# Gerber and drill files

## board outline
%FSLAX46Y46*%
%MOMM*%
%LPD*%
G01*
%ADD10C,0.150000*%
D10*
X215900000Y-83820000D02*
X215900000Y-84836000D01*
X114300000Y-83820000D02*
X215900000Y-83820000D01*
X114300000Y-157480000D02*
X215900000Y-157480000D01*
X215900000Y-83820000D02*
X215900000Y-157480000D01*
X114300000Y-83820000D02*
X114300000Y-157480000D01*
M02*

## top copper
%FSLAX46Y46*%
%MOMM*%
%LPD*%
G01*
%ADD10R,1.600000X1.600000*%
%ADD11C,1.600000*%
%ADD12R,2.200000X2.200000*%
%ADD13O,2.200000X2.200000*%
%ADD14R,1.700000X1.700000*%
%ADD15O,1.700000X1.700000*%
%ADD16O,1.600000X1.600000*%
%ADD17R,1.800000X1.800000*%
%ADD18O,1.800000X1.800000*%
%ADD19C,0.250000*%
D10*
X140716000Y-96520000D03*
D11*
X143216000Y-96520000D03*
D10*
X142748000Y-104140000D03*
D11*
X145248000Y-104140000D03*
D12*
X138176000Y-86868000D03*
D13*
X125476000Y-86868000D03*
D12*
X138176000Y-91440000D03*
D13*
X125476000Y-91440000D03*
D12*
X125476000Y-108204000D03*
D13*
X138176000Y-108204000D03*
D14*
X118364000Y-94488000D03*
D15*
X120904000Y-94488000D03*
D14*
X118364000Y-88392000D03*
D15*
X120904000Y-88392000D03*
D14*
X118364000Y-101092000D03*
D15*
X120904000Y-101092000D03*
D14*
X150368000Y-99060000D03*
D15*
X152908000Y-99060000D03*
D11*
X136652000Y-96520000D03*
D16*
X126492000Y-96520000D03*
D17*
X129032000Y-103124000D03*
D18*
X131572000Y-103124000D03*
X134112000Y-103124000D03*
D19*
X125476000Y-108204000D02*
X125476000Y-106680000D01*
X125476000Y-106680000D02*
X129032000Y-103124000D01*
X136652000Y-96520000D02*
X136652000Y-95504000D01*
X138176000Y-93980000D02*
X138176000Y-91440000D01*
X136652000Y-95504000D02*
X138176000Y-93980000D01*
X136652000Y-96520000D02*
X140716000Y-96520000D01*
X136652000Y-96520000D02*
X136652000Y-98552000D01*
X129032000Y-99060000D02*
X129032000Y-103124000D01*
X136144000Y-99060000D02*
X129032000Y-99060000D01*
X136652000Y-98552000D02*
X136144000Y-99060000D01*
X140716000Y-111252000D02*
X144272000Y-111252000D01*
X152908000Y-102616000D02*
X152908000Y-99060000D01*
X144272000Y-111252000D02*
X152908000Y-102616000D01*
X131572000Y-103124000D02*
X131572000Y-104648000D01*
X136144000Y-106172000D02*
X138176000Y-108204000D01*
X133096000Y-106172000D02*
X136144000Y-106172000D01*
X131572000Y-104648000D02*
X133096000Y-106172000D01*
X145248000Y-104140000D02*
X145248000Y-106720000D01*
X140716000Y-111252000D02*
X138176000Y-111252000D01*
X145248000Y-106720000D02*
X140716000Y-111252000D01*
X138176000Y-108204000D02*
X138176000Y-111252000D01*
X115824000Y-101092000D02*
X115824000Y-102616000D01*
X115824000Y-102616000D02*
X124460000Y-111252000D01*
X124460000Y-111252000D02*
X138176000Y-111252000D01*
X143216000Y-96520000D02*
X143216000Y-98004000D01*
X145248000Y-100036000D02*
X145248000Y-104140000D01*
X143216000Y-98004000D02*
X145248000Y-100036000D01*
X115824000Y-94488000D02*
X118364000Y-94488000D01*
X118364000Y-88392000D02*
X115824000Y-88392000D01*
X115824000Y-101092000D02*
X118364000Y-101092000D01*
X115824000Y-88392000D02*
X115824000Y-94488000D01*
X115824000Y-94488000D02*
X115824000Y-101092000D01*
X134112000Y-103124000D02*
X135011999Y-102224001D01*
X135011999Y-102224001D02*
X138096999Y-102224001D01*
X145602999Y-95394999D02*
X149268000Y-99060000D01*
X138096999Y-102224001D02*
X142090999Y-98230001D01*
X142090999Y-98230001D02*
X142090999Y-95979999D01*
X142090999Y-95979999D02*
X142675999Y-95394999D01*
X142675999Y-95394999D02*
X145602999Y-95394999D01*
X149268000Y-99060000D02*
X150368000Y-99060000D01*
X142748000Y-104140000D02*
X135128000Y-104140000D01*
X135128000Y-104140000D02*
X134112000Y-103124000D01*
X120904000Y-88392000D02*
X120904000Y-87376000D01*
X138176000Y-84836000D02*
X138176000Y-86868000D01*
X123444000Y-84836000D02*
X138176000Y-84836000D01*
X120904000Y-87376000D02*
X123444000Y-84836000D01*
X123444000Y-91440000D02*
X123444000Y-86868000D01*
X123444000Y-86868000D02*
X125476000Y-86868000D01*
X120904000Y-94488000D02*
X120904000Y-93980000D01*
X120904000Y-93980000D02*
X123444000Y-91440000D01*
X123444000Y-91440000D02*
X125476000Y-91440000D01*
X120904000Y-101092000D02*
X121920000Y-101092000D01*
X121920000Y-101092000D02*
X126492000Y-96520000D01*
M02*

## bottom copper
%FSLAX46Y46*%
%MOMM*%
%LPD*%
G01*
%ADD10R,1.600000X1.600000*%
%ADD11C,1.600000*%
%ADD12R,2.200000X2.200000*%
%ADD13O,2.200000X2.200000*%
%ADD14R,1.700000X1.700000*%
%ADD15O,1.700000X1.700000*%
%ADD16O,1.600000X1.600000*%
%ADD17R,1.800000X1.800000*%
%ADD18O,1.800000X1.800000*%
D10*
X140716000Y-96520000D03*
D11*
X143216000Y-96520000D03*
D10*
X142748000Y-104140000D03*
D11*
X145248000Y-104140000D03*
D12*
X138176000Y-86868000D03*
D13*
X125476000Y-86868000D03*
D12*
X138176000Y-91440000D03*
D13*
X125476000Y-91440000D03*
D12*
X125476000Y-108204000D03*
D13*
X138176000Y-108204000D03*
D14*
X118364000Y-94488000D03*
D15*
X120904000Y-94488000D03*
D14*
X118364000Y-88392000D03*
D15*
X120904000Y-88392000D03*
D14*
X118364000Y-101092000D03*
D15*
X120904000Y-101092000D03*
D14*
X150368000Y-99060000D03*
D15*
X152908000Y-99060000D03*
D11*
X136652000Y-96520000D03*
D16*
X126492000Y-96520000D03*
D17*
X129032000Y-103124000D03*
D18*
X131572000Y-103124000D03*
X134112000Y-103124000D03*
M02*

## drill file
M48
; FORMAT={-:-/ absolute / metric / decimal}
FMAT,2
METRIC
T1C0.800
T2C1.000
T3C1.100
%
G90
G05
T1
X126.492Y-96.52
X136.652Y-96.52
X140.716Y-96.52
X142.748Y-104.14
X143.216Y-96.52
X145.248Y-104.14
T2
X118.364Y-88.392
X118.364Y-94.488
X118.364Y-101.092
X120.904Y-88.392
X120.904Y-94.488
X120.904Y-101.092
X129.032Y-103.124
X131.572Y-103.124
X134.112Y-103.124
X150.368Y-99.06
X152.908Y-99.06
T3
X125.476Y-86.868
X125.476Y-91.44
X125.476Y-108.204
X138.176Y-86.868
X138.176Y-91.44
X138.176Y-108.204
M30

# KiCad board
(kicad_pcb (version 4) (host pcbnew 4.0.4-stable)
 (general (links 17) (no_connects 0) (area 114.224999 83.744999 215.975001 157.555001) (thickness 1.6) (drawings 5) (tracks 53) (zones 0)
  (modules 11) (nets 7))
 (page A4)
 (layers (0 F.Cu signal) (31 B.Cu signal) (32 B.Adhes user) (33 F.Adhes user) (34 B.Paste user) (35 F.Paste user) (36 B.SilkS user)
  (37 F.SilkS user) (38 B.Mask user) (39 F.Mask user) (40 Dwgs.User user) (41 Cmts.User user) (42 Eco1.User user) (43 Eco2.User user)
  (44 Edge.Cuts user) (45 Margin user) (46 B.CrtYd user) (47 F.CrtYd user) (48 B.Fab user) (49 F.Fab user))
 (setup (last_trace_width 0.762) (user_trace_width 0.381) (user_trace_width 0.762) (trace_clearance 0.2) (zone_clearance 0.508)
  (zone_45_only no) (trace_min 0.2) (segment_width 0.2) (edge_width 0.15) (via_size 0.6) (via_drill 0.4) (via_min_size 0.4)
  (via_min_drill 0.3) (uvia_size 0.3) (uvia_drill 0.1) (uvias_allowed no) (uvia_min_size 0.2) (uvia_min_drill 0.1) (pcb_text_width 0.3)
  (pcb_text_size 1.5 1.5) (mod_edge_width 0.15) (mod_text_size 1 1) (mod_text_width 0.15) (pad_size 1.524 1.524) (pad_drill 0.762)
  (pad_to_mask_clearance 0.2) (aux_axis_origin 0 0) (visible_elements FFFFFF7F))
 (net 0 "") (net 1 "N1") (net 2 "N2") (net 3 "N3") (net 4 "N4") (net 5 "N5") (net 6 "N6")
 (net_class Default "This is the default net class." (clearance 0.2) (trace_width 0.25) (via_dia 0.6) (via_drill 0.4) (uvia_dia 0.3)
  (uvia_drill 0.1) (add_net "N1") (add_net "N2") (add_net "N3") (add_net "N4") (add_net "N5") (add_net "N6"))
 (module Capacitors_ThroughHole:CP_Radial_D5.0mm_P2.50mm (layer F.Cu) (at 140.716 96.52)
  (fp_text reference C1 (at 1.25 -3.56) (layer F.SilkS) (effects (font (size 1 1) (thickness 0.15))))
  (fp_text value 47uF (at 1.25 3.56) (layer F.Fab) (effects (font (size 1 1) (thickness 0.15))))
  (pad 1 thru_hole rect (at 0 0) (size 1.6 1.6) (drill 0.8) (layers *.Cu *.Mask) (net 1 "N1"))
  (pad 2 thru_hole circle (at 2.5 0) (size 1.6 1.6) (drill 0.8) (layers *.Cu *.Mask) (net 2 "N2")))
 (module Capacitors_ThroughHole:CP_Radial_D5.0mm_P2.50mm (layer F.Cu) (at 142.748 104.14)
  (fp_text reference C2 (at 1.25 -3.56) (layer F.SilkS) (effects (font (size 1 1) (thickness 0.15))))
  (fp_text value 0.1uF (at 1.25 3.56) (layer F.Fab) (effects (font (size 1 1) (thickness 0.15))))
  (pad 1 thru_hole rect (at 0 0) (size 1.6 1.6) (drill 0.8) (layers *.Cu *.Mask) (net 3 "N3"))
  (pad 2 thru_hole circle (at 2.5 0) (size 1.6 1.6) (drill 0.8) (layers *.Cu *.Mask) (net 2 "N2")))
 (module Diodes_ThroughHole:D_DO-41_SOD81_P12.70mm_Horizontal (layer F.Cu) (at 138.176 86.868 180)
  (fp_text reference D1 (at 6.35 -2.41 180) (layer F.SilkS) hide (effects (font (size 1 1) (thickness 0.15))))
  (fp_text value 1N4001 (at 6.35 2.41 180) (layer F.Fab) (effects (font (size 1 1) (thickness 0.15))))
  (pad 1 thru_hole rect (at 0 0 180) (size 2.2 2.2) (drill 1.1) (layers *.Cu *.Mask) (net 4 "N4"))
  (pad 2 thru_hole oval (at 12.7 0 180) (size 2.2 2.2) (drill 1.1) (layers *.Cu *.Mask) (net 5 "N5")))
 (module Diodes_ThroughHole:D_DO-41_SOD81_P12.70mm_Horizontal (layer F.Cu) (at 138.176 91.44 180)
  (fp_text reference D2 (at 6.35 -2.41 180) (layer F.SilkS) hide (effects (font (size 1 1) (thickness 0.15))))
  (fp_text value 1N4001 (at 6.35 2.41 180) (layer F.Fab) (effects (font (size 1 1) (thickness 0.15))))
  (pad 1 thru_hole rect (at 0 0 180) (size 2.2 2.2) (drill 1.1) (layers *.Cu *.Mask) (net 1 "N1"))
  (pad 2 thru_hole oval (at 12.7 0 180) (size 2.2 2.2) (drill 1.1) (layers *.Cu *.Mask) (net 5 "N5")))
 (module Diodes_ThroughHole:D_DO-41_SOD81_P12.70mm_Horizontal (layer F.Cu) (at 125.476 108.204)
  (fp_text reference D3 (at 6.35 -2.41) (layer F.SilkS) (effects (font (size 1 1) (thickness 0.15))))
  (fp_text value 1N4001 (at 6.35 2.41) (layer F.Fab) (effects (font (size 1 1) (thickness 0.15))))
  (pad 1 thru_hole rect (at 0 0) (size 2.2 2.2) (drill 1.1) (layers *.Cu *.Mask) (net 1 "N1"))
  (pad 2 thru_hole oval (at 12.7 0) (size 2.2 2.2) (drill 1.1) (layers *.Cu *.Mask) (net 2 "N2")))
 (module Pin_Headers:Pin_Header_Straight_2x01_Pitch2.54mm (layer F.Cu) (at 118.364 94.488)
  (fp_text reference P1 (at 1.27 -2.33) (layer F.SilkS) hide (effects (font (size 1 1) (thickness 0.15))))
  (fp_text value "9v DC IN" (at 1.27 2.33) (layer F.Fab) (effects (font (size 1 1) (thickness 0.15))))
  (pad 1 thru_hole rect (at 0 0) (size 1.7 1.7) (drill 1) (layers *.Cu *.Mask) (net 2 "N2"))
  (pad 2 thru_hole oval (at 2.54 0) (size 1.7 1.7) (drill 1) (layers *.Cu *.Mask) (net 5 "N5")))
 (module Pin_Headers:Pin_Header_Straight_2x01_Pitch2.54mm (layer F.Cu) (at 118.364 88.392)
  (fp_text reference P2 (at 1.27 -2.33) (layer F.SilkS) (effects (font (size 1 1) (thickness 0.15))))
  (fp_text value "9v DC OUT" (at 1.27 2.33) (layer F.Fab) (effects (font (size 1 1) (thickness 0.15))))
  (pad 1 thru_hole rect (at 0 0) (size 1.7 1.7) (drill 1) (layers *.Cu *.Mask) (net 2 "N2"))
  (pad 2 thru_hole oval (at 2.54 0) (size 1.7 1.7) (drill 1) (layers *.Cu *.Mask) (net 4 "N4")))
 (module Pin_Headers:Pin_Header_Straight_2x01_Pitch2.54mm (layer F.Cu) (at 118.364 101.092)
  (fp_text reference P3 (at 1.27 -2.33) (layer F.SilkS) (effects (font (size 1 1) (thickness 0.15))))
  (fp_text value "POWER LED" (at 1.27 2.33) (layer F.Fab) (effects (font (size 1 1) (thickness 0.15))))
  (pad 1 thru_hole rect (at 0 0) (size 1.7 1.7) (drill 1) (layers *.Cu *.Mask) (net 2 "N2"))
  (pad 2 thru_hole oval (at 2.54 0) (size 1.7 1.7) (drill 1) (layers *.Cu *.Mask) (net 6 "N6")))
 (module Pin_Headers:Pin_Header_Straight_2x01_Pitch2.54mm (layer F.Cu) (at 150.368 99.06)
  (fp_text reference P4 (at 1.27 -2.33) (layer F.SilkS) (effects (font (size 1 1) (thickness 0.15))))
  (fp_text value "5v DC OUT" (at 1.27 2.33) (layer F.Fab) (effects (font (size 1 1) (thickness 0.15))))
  (pad 1 thru_hole rect (at 0 0) (size 1.7 1.7) (drill 1) (layers *.Cu *.Mask) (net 3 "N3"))
  (pad 2 thru_hole oval (at 2.54 0) (size 1.7 1.7) (drill 1) (layers *.Cu *.Mask) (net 2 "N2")))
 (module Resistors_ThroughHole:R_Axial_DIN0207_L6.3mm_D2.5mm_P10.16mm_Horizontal (layer F.Cu) (at 136.652 96.52 180)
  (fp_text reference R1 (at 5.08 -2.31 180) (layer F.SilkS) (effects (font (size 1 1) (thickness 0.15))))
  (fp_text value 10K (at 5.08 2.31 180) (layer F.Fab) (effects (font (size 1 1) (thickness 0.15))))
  (pad 1 thru_hole circle (at 0 0 180) (size 1.6 1.6) (drill 0.8) (layers *.Cu *.Mask) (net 1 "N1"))
  (pad 2 thru_hole oval (at 10.16 0 180) (size 1.6 1.6) (drill 0.8) (layers *.Cu *.Mask) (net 6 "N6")))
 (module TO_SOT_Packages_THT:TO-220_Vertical (layer F.Cu) (at 129.032 103.124)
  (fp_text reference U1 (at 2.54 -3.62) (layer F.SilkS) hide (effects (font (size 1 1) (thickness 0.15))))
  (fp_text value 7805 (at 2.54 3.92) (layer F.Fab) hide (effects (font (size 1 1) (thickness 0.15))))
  (pad 1 thru_hole rect (at 0 0) (size 1.8 1.8) (drill 1) (layers *.Cu *.Mask) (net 1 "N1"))
  (pad 2 thru_hole oval (at 2.54 0) (size 1.8 1.8) (drill 1) (layers *.Cu *.Mask) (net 2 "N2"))
  (pad 3 thru_hole oval (at 5.08 0) (size 1.8 1.8) (drill 1) (layers *.Cu *.Mask) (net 3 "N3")))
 (gr_line (start 215.9 83.82) (end 215.9 84.836) (angle 90) (layer Edge.Cuts) (width 0.15))
 (gr_line (start 114.3 83.82) (end 215.9 83.82) (angle 90) (layer Edge.Cuts) (width 0.15))
 (gr_line (start 114.3 157.48) (end 215.9 157.48) (angle 90) (layer Edge.Cuts) (width 0.15))
 (gr_line (start 215.9 83.82) (end 215.9 157.48) (angle 90) (layer Edge.Cuts) (width 0.15))
 (gr_line (start 114.3 83.82) (end 114.3 157.48) (angle 90) (layer Edge.Cuts) (width 0.15))
 (segment (start 125.476 108.204) (end 125.476 106.68) (width 0.25) (layer F.Cu) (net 1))
 (segment (start 125.476 106.68) (end 129.032 103.124) (width 0.25) (layer F.Cu) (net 1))
 (segment (start 136.652 96.52) (end 136.652 95.504) (width 0.25) (layer F.Cu) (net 1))
 (segment (start 138.176 93.98) (end 138.176 91.44) (width 0.25) (layer F.Cu) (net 1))
 (segment (start 136.652 95.504) (end 138.176 93.98) (width 0.25) (layer F.Cu) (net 1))
 (segment (start 136.652 96.52) (end 140.716 96.52) (width 0.25) (layer F.Cu) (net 1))
 (segment (start 136.652 96.52) (end 136.652 98.552) (width 0.25) (layer F.Cu) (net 1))
 (segment (start 129.032 99.06) (end 129.032 103.124) (width 0.25) (layer F.Cu) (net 1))
 (segment (start 136.144 99.06) (end 129.032 99.06) (width 0.25) (layer F.Cu) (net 1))
 (segment (start 136.652 98.552) (end 136.144 99.06) (width 0.25) (layer F.Cu) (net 1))
 (segment (start 140.716 111.252) (end 144.272 111.252) (width 0.25) (layer F.Cu) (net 2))
 (segment (start 152.908 102.616) (end 152.908 99.06) (width 0.25) (layer F.Cu) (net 2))
 (segment (start 144.272 111.252) (end 152.908 102.616) (width 0.25) (layer F.Cu) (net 2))
 (segment (start 131.572 103.124) (end 131.572 104.648) (width 0.25) (layer F.Cu) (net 2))
 (segment (start 136.144 106.172) (end 138.176 108.204) (width 0.25) (layer F.Cu) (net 2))
 (segment (start 133.096 106.172) (end 136.144 106.172) (width 0.25) (layer F.Cu) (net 2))
 (segment (start 131.572 104.648) (end 133.096 106.172) (width 0.25) (layer F.Cu) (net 2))
 (segment (start 145.248 104.14) (end 145.248 106.72) (width 0.25) (layer F.Cu) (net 2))
 (segment (start 140.716 111.252) (end 138.176 111.252) (width 0.25) (layer F.Cu) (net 2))
 (segment (start 145.248 106.72) (end 140.716 111.252) (width 0.25) (layer F.Cu) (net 2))
 (segment (start 138.176 108.204) (end 138.176 111.252) (width 0.25) (layer F.Cu) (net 2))
 (segment (start 115.824 101.092) (end 115.824 102.616) (width 0.25) (layer F.Cu) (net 2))
 (segment (start 115.824 102.616) (end 124.46 111.252) (width 0.25) (layer F.Cu) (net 2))
 (segment (start 124.46 111.252) (end 138.176 111.252) (width 0.25) (layer F.Cu) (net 2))
 (segment (start 143.216 96.52) (end 143.216 98.004) (width 0.25) (layer F.Cu) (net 2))
 (segment (start 145.248 100.036) (end 145.248 104.14) (width 0.25) (layer F.Cu) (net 2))
 (segment (start 143.216 98.004) (end 145.248 100.036) (width 0.25) (layer F.Cu) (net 2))
 (segment (start 115.824 94.488) (end 118.364 94.488) (width 0.25) (layer F.Cu) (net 2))
 (segment (start 118.364 88.392) (end 115.824 88.392) (width 0.25) (layer F.Cu) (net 2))
 (segment (start 115.824 101.092) (end 118.364 101.092) (width 0.25) (layer F.Cu) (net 2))
 (segment (start 115.824 88.392) (end 115.824 94.488) (width 0.25) (layer F.Cu) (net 2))
 (segment (start 115.824 94.488) (end 115.824 101.092) (width 0.25) (layer F.Cu) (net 2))
 (segment (start 134.112 103.124) (end 135.011999 102.224001) (width 0.25) (layer F.Cu) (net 3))
 (segment (start 135.011999 102.224001) (end 138.096999 102.224001) (width 0.25) (layer F.Cu) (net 3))
 (segment (start 145.602999 95.394999) (end 149.268 99.06) (width 0.25) (layer F.Cu) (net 3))
 (segment (start 138.096999 102.224001) (end 142.090999 98.230001) (width 0.25) (layer F.Cu) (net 3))
 (segment (start 142.090999 98.230001) (end 142.090999 95.979999) (width 0.25) (layer F.Cu) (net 3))
 (segment (start 142.090999 95.979999) (end 142.675999 95.394999) (width 0.25) (layer F.Cu) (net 3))
 (segment (start 142.675999 95.394999) (end 145.602999 95.394999) (width 0.25) (layer F.Cu) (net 3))
 (segment (start 149.268 99.06) (end 150.368 99.06) (width 0.25) (layer F.Cu) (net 3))
 (segment (start 142.748 104.14) (end 135.128 104.14) (width 0.25) (layer F.Cu) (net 3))
 (segment (start 135.128 104.14) (end 134.112 103.124) (width 0.25) (layer F.Cu) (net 3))
 (segment (start 120.904 88.392) (end 120.904 87.376) (width 0.25) (layer F.Cu) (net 4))
 (segment (start 138.176 84.836) (end 138.176 86.868) (width 0.25) (layer F.Cu) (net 4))
 (segment (start 123.444 84.836) (end 138.176 84.836) (width 0.25) (layer F.Cu) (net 4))
 (segment (start 120.904 87.376) (end 123.444 84.836) (width 0.25) (layer F.Cu) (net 4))
 (segment (start 123.444 91.44) (end 123.444 86.868) (width 0.25) (layer F.Cu) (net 5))
 (segment (start 123.444 86.868) (end 125.476 86.868) (width 0.25) (layer F.Cu) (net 5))
 (segment (start 120.904 94.488) (end 120.904 93.98) (width 0.25) (layer F.Cu) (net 5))
 (segment (start 120.904 93.98) (end 123.444 91.44) (width 0.25) (layer F.Cu) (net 5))
 (segment (start 123.444 91.44) (end 125.476 91.44) (width 0.25) (layer F.Cu) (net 5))
 (segment (start 120.904 101.092) (end 121.92 101.092) (width 0.25) (layer F.Cu) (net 6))
 (segment (start 121.92 101.092) (end 126.492 96.52) (width 0.25) (layer F.Cu) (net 6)))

